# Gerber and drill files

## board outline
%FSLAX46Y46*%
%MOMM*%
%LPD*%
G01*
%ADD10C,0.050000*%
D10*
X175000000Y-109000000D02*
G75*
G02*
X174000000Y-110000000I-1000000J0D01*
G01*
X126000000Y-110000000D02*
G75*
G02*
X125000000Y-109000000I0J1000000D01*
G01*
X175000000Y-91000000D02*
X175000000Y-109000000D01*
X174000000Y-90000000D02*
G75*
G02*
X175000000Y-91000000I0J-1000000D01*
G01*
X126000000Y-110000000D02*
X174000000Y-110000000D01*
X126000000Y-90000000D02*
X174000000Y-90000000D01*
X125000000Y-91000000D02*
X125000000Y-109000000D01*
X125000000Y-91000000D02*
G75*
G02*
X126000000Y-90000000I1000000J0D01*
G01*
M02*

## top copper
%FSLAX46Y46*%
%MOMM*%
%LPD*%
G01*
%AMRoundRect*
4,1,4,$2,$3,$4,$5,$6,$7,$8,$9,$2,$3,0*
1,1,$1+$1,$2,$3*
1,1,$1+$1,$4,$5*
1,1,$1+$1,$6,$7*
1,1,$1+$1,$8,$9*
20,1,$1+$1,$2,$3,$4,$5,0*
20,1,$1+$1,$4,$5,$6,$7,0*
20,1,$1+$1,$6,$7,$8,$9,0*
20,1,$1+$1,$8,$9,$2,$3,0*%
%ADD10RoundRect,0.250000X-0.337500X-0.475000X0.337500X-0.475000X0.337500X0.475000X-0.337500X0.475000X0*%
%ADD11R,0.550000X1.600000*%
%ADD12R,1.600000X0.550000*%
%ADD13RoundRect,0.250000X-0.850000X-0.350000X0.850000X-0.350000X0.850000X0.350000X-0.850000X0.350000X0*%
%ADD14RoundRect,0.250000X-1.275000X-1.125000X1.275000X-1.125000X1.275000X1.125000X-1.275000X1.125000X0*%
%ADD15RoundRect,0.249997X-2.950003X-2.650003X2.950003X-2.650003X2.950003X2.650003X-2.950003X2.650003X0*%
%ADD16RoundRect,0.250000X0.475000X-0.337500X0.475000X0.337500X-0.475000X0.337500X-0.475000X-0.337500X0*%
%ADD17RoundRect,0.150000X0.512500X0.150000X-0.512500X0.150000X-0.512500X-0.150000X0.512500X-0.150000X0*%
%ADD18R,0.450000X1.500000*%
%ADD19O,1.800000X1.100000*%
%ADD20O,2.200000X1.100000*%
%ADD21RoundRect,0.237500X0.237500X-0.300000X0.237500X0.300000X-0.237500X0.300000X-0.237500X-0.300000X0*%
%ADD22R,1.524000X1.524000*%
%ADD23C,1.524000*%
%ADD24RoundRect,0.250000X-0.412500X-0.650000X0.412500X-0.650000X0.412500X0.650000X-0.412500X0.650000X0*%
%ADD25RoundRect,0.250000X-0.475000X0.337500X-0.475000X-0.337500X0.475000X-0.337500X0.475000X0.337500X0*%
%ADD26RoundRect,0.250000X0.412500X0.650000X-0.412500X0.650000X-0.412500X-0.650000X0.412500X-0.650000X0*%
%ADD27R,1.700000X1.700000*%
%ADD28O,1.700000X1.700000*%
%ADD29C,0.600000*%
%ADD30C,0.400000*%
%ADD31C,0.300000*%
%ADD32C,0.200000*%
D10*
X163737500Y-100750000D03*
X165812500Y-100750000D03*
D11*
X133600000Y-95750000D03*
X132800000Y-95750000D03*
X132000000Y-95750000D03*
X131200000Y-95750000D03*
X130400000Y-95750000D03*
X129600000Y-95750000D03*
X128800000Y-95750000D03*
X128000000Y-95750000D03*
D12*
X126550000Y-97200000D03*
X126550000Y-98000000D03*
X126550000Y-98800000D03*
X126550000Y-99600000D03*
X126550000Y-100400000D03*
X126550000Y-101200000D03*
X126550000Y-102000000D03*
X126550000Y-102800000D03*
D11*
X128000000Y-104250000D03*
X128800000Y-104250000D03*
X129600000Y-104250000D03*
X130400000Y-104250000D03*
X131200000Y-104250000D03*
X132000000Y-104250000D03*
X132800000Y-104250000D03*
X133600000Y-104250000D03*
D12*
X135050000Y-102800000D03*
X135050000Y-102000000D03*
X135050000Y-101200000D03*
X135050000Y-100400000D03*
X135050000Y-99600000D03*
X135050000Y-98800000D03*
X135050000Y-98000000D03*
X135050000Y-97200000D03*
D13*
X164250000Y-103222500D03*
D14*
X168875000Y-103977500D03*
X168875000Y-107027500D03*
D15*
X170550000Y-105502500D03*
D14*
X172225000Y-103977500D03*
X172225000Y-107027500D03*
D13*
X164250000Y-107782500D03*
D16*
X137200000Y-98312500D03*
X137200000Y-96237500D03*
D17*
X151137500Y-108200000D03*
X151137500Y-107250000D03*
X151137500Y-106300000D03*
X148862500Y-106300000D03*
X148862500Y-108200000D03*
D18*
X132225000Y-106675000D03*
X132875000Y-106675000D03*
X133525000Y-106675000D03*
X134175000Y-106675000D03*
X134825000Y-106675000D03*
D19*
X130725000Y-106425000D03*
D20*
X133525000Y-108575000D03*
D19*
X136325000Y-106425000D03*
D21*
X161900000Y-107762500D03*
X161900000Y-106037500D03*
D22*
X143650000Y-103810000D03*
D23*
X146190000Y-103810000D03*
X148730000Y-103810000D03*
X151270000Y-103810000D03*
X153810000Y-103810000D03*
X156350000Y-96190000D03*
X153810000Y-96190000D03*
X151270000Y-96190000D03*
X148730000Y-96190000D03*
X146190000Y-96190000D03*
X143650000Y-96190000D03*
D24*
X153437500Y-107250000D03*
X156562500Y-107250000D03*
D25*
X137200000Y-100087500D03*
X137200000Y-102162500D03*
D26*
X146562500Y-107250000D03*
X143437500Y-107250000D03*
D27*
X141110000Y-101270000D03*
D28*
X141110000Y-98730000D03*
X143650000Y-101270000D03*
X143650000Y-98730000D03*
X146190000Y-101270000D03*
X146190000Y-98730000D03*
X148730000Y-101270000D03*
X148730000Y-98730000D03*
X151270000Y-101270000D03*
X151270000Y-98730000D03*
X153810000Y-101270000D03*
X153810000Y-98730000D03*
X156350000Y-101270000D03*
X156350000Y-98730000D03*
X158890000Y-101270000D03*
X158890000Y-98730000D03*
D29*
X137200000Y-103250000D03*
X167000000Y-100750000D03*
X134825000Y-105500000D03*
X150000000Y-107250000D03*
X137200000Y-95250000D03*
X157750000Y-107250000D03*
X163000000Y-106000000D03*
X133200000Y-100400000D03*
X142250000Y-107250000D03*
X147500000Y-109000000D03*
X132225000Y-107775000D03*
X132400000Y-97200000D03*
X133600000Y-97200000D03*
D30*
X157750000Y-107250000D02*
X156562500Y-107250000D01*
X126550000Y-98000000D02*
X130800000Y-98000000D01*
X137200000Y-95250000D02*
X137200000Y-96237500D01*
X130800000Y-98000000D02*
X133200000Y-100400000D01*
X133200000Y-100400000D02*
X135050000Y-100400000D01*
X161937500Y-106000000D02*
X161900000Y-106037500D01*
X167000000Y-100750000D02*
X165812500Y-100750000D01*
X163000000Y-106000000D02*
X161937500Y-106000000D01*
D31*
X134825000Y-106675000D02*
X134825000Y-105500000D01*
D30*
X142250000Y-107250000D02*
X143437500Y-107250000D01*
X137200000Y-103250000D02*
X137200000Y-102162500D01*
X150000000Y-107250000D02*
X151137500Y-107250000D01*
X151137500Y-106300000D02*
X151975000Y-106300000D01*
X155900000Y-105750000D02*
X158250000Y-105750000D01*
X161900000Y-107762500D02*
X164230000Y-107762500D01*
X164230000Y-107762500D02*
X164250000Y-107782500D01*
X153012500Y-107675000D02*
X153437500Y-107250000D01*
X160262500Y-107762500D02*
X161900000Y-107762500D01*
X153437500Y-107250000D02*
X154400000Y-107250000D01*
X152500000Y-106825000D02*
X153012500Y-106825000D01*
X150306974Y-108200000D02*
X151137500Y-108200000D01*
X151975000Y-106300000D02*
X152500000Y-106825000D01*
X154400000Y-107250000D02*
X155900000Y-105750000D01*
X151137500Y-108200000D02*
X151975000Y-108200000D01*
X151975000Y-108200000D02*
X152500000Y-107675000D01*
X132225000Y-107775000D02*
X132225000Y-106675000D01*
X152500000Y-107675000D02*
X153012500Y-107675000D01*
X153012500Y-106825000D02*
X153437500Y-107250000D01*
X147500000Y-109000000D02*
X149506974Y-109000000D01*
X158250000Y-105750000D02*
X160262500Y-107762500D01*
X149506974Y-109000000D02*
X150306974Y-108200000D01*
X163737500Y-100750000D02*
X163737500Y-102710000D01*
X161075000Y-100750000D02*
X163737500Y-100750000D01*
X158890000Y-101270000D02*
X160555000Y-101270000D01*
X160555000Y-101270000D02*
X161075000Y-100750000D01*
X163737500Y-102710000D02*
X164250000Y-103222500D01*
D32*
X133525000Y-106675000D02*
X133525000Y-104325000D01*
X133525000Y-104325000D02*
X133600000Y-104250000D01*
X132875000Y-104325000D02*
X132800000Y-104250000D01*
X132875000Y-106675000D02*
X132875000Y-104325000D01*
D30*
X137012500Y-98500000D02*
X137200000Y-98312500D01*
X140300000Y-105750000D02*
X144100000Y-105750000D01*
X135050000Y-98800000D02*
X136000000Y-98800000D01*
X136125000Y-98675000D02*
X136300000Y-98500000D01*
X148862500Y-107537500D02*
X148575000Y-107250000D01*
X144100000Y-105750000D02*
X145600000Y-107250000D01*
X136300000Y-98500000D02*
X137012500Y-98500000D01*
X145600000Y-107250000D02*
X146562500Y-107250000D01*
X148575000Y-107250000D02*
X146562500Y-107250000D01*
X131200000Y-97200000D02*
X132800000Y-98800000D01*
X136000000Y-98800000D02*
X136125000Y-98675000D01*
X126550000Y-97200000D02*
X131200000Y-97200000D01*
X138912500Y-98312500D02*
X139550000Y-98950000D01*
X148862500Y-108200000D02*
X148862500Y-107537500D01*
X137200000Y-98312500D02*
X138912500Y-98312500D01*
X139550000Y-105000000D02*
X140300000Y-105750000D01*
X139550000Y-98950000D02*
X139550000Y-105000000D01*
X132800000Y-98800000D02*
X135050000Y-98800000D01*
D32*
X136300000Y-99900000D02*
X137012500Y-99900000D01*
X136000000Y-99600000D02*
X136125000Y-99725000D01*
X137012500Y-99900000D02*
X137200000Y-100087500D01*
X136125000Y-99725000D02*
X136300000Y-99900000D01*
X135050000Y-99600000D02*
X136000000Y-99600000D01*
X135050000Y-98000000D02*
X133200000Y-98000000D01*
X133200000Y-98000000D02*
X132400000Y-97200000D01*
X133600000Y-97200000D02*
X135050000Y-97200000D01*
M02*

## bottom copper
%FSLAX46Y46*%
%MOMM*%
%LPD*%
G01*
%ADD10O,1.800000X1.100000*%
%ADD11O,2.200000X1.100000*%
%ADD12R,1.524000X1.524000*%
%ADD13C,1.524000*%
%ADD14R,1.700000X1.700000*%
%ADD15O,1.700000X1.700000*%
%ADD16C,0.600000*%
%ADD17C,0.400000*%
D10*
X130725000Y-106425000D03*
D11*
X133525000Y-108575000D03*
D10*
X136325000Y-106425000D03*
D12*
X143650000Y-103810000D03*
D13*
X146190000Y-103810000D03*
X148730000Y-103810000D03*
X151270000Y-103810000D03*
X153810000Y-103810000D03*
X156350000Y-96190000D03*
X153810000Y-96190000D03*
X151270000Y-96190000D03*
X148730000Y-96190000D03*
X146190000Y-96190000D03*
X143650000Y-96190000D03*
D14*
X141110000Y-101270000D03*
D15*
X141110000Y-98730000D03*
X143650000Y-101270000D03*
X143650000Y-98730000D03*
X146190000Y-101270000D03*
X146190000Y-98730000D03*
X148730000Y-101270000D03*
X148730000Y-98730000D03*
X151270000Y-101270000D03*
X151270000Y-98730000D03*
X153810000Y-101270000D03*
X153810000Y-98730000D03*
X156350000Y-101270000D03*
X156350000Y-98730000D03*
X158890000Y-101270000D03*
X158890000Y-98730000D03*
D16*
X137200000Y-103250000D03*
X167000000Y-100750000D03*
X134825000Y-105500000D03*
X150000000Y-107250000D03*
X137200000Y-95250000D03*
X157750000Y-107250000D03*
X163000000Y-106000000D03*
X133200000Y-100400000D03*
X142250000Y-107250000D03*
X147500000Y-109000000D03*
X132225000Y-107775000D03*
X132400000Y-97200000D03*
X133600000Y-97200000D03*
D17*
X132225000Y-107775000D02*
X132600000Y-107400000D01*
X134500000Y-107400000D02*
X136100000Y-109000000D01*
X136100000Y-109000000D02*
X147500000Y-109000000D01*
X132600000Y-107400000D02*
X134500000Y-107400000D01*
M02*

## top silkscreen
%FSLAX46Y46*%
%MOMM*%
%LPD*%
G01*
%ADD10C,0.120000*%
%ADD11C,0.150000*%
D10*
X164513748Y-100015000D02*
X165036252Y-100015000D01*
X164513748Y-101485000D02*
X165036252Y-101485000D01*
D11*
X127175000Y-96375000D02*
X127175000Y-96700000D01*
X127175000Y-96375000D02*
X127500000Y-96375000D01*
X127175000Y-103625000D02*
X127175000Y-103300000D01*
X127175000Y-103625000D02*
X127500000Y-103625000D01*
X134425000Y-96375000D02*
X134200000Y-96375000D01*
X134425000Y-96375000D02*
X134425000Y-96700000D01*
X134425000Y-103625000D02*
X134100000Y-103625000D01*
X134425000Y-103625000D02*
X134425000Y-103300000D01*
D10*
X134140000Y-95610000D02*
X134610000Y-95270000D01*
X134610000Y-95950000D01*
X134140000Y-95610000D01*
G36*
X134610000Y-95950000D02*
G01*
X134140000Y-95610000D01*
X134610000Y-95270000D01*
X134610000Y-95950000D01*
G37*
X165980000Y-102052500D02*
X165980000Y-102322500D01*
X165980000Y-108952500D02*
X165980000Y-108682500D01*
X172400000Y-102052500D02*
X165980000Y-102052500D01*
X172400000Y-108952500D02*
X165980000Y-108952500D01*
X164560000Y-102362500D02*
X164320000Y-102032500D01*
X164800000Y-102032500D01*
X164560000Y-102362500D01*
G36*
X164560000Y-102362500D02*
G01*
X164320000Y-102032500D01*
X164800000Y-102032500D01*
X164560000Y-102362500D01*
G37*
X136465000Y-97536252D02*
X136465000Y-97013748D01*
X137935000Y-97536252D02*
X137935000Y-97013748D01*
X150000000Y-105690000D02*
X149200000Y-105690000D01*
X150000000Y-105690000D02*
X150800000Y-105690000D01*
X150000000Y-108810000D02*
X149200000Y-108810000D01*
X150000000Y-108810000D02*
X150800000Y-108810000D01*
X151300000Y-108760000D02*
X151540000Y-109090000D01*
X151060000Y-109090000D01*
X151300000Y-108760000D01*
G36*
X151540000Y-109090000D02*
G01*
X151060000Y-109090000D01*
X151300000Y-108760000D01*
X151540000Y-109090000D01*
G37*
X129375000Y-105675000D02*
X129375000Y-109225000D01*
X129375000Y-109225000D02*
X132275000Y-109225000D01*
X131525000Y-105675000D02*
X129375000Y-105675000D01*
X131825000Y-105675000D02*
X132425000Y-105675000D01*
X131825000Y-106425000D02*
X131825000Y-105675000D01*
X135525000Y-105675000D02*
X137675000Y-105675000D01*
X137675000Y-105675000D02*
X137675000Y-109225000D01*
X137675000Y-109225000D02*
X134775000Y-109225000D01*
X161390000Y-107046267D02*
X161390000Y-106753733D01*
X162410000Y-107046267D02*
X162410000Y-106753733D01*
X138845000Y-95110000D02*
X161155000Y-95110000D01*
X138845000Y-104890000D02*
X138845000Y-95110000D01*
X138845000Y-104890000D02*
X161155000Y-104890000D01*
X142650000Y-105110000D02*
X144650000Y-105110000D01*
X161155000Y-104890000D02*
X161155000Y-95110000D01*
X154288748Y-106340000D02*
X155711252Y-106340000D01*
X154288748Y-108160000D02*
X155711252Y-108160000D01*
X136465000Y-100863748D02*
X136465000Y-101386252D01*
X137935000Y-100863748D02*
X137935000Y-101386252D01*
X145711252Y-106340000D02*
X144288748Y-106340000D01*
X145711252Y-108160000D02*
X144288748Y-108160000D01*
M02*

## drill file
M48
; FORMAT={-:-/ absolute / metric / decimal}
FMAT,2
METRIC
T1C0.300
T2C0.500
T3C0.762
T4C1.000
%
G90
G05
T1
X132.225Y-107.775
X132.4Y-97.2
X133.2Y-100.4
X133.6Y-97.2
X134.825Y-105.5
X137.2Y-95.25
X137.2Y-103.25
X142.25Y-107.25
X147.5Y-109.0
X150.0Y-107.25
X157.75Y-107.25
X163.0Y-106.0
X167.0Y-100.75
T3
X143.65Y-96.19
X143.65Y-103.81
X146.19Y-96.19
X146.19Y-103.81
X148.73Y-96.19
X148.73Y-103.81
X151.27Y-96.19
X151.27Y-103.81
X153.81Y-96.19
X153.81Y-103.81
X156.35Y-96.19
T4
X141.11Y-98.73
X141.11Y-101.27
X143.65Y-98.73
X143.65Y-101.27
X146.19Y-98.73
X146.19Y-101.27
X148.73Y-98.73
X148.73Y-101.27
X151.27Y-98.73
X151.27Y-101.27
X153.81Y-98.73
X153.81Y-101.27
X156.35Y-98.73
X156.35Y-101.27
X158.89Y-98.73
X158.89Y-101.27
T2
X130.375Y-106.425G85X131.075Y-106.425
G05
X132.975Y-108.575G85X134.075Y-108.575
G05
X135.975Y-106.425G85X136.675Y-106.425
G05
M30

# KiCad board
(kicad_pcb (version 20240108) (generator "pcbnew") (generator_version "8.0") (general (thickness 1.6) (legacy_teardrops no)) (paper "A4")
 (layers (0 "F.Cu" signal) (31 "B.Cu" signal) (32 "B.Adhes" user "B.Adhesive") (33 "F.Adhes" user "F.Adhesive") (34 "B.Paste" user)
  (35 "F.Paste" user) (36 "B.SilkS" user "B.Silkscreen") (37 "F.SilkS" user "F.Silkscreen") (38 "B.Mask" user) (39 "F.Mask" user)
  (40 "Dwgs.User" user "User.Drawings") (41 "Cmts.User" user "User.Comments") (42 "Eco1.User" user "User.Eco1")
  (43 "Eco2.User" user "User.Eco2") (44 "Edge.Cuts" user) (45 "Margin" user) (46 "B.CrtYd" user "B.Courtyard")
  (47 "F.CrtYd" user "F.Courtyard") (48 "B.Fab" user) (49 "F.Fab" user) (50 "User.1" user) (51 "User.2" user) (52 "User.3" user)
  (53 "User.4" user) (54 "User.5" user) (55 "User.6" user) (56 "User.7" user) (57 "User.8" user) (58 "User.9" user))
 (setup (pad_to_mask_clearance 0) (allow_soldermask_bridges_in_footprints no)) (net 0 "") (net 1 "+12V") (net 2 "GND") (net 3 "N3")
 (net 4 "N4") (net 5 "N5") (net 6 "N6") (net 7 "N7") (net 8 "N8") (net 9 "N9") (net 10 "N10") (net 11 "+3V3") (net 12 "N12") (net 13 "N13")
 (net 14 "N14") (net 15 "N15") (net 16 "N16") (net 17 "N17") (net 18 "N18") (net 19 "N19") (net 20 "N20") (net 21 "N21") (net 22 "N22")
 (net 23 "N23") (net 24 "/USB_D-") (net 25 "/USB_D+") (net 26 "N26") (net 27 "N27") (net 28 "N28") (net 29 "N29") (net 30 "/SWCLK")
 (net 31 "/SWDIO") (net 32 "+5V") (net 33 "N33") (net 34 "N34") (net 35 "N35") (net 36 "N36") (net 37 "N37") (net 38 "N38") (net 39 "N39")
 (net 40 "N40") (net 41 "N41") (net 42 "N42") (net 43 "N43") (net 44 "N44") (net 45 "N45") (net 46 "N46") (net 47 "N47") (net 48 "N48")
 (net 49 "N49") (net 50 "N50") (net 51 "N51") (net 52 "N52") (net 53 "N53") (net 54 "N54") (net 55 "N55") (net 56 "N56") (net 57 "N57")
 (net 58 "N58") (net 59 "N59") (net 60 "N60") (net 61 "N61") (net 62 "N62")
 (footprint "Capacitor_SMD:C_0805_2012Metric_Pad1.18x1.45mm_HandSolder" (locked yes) (layer "F.Cu") (at 164.775 100.75)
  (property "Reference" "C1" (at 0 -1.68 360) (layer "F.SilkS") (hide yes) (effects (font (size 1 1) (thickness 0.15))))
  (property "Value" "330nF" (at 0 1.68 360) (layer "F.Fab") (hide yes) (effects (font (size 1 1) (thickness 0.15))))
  (fp_line (start -0.261252 -0.735) (end 0.261252 -0.735) (stroke (width 0.12) (type solid)) (layer "F.SilkS"))
  (fp_line (start -0.261252 0.735) (end 0.261252 0.735) (stroke (width 0.12) (type solid)) (layer "F.SilkS"))
  (pad "1" smd roundrect (at -1.0375 0) (size 1.175 1.45) (layers "F.Cu" "F.Paste" "F.Mask") (roundrect_rratio 0.212766) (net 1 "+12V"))
  (pad "2" smd roundrect (at 1.0375 0) (size 1.175 1.45) (layers "F.Cu" "F.Paste" "F.Mask") (roundrect_rratio 0.212766) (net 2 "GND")))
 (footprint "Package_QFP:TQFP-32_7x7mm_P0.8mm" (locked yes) (layer "F.Cu") (at 130.8 100 -90)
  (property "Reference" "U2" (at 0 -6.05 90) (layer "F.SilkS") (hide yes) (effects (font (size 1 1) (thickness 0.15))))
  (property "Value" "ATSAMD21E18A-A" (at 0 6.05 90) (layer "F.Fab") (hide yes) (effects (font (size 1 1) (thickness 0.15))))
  (fp_line (start -3.625 3.625) (end -3.3 3.625) (stroke (width 0.15) (type solid)) (layer "F.SilkS"))
  (fp_line (start -3.625 3.625) (end -3.625 3.3) (stroke (width 0.15) (type solid)) (layer "F.SilkS"))
  (fp_line (start 3.625 3.625) (end 3.3 3.625) (stroke (width 0.15) (type solid)) (layer "F.SilkS"))
  (fp_line (start 3.625 3.625) (end 3.625 3.3) (stroke (width 0.15) (type solid)) (layer "F.SilkS"))
  (fp_line (start -3.625 -3.625) (end -3.625 -3.4) (stroke (width 0.15) (type solid)) (layer "F.SilkS"))
  (fp_line (start -3.625 -3.625) (end -3.3 -3.625) (stroke (width 0.15) (type solid)) (layer "F.SilkS"))
  (fp_line (start 3.625 -3.625) (end 3.625 -3.3) (stroke (width 0.15) (type solid)) (layer "F.SilkS"))
  (fp_line (start 3.625 -3.625) (end 3.3 -3.625) (stroke (width 0.15) (type solid)) (layer "F.SilkS"))
  (fp_poly
   (pts (xy -4.39 -3.34) (xy -4.73 -3.81) (xy -4.05 -3.81) (xy -4.39 -3.34)) (stroke (width 0.12) (type solid)) (fill solid)
   (layer "F.SilkS"))
  (pad "1" smd rect (at -4.25 -2.8 270) (size 1.6 0.55) (layers "F.Cu" "F.Paste" "F.Mask") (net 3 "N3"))
  (pad "2" smd rect (at -4.25 -2 270) (size 1.6 0.55) (layers "F.Cu" "F.Paste" "F.Mask") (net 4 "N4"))
  (pad "3" smd rect (at -4.25 -1.2 270) (size 1.6 0.55) (layers "F.Cu" "F.Paste" "F.Mask") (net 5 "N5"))
  (pad "4" smd rect (at -4.25 -0.4 270) (size 1.6 0.55) (layers "F.Cu" "F.Paste" "F.Mask") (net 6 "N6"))
  (pad "5" smd rect (at -4.25 0.4 270) (size 1.6 0.55) (layers "F.Cu" "F.Paste" "F.Mask") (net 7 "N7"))
  (pad "6" smd rect (at -4.25 1.2 270) (size 1.6 0.55) (layers "F.Cu" "F.Paste" "F.Mask") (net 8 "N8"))
  (pad "7" smd rect (at -4.25 2 270) (size 1.6 0.55) (layers "F.Cu" "F.Paste" "F.Mask") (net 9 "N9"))
  (pad "8" smd rect (at -4.25 2.8 270) (size 1.6 0.55) (layers "F.Cu" "F.Paste" "F.Mask") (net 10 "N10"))
  (pad "9" smd rect (at -2.8 4.25) (size 1.6 0.55) (layers "F.Cu" "F.Paste" "F.Mask") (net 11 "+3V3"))
  (pad "10" smd rect (at -2 4.25) (size 1.6 0.55) (layers "F.Cu" "F.Paste" "F.Mask") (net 2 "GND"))
  (pad "11" smd rect (at -1.2 4.25) (size 1.6 0.55) (layers "F.Cu" "F.Paste" "F.Mask") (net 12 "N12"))
  (pad "12" smd rect (at -0.4 4.25) (size 1.6 0.55) (layers "F.Cu" "F.Paste" "F.Mask") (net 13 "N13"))
  (pad "13" smd rect (at 0.4 4.25) (size 1.6 0.55) (layers "F.Cu" "F.Paste" "F.Mask") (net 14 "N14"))
  (pad "14" smd rect (at 1.2 4.25) (size 1.6 0.55) (layers "F.Cu" "F.Paste" "F.Mask") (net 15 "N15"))
  (pad "15" smd rect (at 2 4.25) (size 1.6 0.55) (layers "F.Cu" "F.Paste" "F.Mask") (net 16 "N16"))
  (pad "16" smd rect (at 2.8 4.25) (size 1.6 0.55) (layers "F.Cu" "F.Paste" "F.Mask") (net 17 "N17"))
  (pad "17" smd rect (at 4.25 2.8 270) (size 1.6 0.55) (layers "F.Cu" "F.Paste" "F.Mask") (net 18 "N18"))
  (pad "18" smd rect (at 4.25 2 270) (size 1.6 0.55) (layers "F.Cu" "F.Paste" "F.Mask") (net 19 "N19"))
  (pad "19" smd rect (at 4.25 1.2 270) (size 1.6 0.55) (layers "F.Cu" "F.Paste" "F.Mask") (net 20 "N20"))
  (pad "20" smd rect (at 4.25 0.4 270) (size 1.6 0.55) (layers "F.Cu" "F.Paste" "F.Mask") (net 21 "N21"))
  (pad "21" smd rect (at 4.25 -0.4 270) (size 1.6 0.55) (layers "F.Cu" "F.Paste" "F.Mask") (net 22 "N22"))
  (pad "22" smd rect (at 4.25 -1.2 270) (size 1.6 0.55) (layers "F.Cu" "F.Paste" "F.Mask") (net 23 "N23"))
  (pad "23" smd rect (at 4.25 -2 270) (size 1.6 0.55) (layers "F.Cu" "F.Paste" "F.Mask") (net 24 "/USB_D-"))
  (pad "24" smd rect (at 4.25 -2.8 270) (size 1.6 0.55) (layers "F.Cu" "F.Paste" "F.Mask") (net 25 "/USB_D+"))
  (pad "25" smd rect (at 2.8 -4.25) (size 1.6 0.55) (layers "F.Cu" "F.Paste" "F.Mask") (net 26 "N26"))
  (pad "26" smd rect (at 2 -4.25) (size 1.6 0.55) (layers "F.Cu" "F.Paste" "F.Mask") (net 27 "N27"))
  (pad "27" smd rect (at 1.2 -4.25) (size 1.6 0.55) (layers "F.Cu" "F.Paste" "F.Mask") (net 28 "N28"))
  (pad "28" smd rect (at 0.4 -4.25) (size 1.6 0.55) (layers "F.Cu" "F.Paste" "F.Mask") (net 2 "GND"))
  (pad "29" smd rect (at -0.4 -4.25) (size 1.6 0.55) (layers "F.Cu" "F.Paste" "F.Mask") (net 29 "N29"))
  (pad "30" smd rect (at -1.2 -4.25) (size 1.6 0.55) (layers "F.Cu" "F.Paste" "F.Mask") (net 11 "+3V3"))
  (pad "31" smd rect (at -2 -4.25) (size 1.6 0.55) (layers "F.Cu" "F.Paste" "F.Mask") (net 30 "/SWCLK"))
  (pad "32" smd rect (at -2.8 -4.25) (size 1.6 0.55) (layers "F.Cu" "F.Paste" "F.Mask") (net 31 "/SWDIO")))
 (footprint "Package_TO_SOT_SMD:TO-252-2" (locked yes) (layer "F.Cu") (at 169.29 105.5025)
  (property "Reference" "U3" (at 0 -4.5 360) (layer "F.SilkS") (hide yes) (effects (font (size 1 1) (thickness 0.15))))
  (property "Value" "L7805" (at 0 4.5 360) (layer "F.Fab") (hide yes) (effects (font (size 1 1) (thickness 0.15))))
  (fp_line (start -3.31 -3.45) (end -3.31 -3.18) (stroke (width 0.12) (type solid)) (layer "F.SilkS"))
  (fp_line (start -3.31 3.45) (end -3.31 3.18) (stroke (width 0.12) (type solid)) (layer "F.SilkS"))
  (fp_line (start 3.11 -3.45) (end -3.31 -3.45) (stroke (width 0.12) (type solid)) (layer "F.SilkS"))
  (fp_line (start 3.11 3.45) (end -3.31 3.45) (stroke (width 0.12) (type solid)) (layer "F.SilkS"))
  (fp_poly
   (pts (xy -4.73 -3.14) (xy -4.97 -3.47) (xy -4.49 -3.47) (xy -4.73 -3.14)) (stroke (width 0.12) (type solid)) (fill solid)
   (layer "F.SilkS"))
  (pad "1" smd roundrect (at -5.04 -2.28) (size 2.2 1.2) (layers "F.Cu" "F.Paste" "F.Mask") (roundrect_rratio 0.208333) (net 1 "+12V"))
  (pad "2" smd roundrect (at -0.415 -1.525) (size 3.05 2.75) (layers "F.Cu" "F.Paste") (roundrect_rratio 0.090909) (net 2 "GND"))
  (pad "2" smd roundrect (at -0.415 1.525) (size 3.05 2.75) (layers "F.Cu" "F.Paste") (roundrect_rratio 0.090909) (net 2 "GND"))
  (pad "2" smd roundrect (at 1.26 0) (size 6.4 5.8) (layers "F.Cu" "F.Mask") (roundrect_rratio 0.043103) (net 2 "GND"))
  (pad "2" smd roundrect (at 2.935 -1.525) (size 3.05 2.75) (layers "F.Cu" "F.Paste") (roundrect_rratio 0.090909) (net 2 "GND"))
  (pad "2" smd roundrect (at 2.935 1.525) (size 3.05 2.75) (layers "F.Cu" "F.Paste") (roundrect_rratio 0.090909) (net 2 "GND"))
  (pad "3" smd roundrect (at -5.04 2.28) (size 2.2 1.2) (layers "F.Cu" "F.Paste" "F.Mask") (roundrect_rratio 0.208333) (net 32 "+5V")))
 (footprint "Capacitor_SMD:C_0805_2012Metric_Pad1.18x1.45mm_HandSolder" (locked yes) (layer "F.Cu") (at 137.2 97.275 90)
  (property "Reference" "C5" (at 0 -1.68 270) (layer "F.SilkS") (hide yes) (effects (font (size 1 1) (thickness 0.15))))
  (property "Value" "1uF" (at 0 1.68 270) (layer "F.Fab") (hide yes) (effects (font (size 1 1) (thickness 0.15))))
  (fp_line (start -0.261252 -0.735) (end 0.261252 -0.735) (stroke (width 0.12) (type solid)) (layer "F.SilkS"))
  (fp_line (start -0.261252 0.735) (end 0.261252 0.735) (stroke (width 0.12) (type solid)) (layer "F.SilkS"))
  (pad "1" smd roundrect (at -1.0375 0 90) (size 1.175 1.45) (layers "F.Cu" "F.Paste" "F.Mask") (roundrect_rratio 0.212766) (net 11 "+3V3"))
  (pad "2" smd roundrect (at 1.0375 0 90) (size 1.175 1.45) (layers "F.Cu" "F.Paste" "F.Mask") (roundrect_rratio 0.212766) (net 2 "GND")))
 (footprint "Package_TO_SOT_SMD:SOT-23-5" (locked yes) (layer "F.Cu") (at 150 107.25 180)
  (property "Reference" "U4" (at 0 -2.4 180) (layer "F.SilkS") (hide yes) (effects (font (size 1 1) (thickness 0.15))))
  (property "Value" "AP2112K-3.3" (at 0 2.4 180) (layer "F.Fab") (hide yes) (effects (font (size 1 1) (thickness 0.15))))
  (fp_line (start 0 1.56) (end 0.8 1.56) (stroke (width 0.12) (type solid)) (layer "F.SilkS"))
  (fp_line (start 0 1.56) (end -0.8 1.56) (stroke (width 0.12) (type solid)) (layer "F.SilkS"))
  (fp_line (start 0 -1.56) (end 0.8 -1.56) (stroke (width 0.12) (type solid)) (layer "F.SilkS"))
  (fp_line (start 0 -1.56) (end -0.8 -1.56) (stroke (width 0.12) (type solid)) (layer "F.SilkS"))
  (fp_poly
   (pts (xy -1.3 -1.51) (xy -1.54 -1.84) (xy -1.06 -1.84) (xy -1.3 -1.51)) (stroke (width 0.12) (type solid)) (fill solid) (layer "F.SilkS"))
  (pad "1" smd roundrect (at -1.1375 -0.95 180) (size 1.325 0.6) (layers "F.Cu" "F.Paste" "F.Mask") (roundrect_rratio 0.25) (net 32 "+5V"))
  (pad "2" smd roundrect (at -1.1375 0 180) (size 1.325 0.6) (layers "F.Cu" "F.Paste" "F.Mask") (roundrect_rratio 0.25) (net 2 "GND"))
  (pad "3" smd roundrect (at -1.1375 0.95 180) (size 1.325 0.6) (layers "F.Cu" "F.Paste" "F.Mask") (roundrect_rratio 0.25) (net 32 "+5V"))
  (pad "4" smd roundrect (at 1.1375 0.95 180) (size 1.325 0.6) (layers "F.Cu" "F.Paste" "F.Mask") (roundrect_rratio 0.25) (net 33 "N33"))
  (pad "5" smd roundrect (at 1.1375 -0.95 180) (size 1.325 0.6) (layers "F.Cu" "F.Paste" "F.Mask") (roundrect_rratio 0.25) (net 11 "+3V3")))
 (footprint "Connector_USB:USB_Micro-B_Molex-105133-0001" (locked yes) (layer "F.Cu") (at 133.525 107.5)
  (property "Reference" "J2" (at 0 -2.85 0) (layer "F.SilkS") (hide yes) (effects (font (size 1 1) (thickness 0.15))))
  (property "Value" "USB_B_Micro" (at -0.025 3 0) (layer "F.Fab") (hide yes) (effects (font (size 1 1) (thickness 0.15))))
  (fp_line (start -4.15 -1.825) (end -4.15 1.725) (stroke (width 0.12) (type solid)) (layer "F.SilkS"))
  (fp_line (start -4.15 1.725) (end -1.25 1.725) (stroke (width 0.12) (type solid)) (layer "F.SilkS"))
  (fp_line (start -2 -1.825) (end -4.15 -1.825) (stroke (width 0.12) (type solid)) (layer "F.SilkS"))
  (fp_line (start -1.7 -1.825) (end -1.1 -1.825) (stroke (width 0.12) (type solid)) (layer "F.SilkS"))
  (fp_line (start -1.7 -1.075) (end -1.7 -1.825) (stroke (width 0.12) (type solid)) (layer "F.SilkS"))
  (fp_line (start 2 -1.825) (end 4.15 -1.825) (stroke (width 0.12) (type solid)) (layer "F.SilkS"))
  (fp_line (start 4.15 -1.825) (end 4.15 1.725) (stroke (width 0.12) (type solid)) (layer "F.SilkS"))
  (fp_line (start 4.15 1.725) (end 1.25 1.725) (stroke (width 0.12) (type solid)) (layer "F.SilkS"))
  (pad "1" smd rect (at -1.3 -0.825) (size 0.45 1.5) (layers "F.Cu" "F.Paste" "F.Mask") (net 32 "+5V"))
  (pad "2" smd rect (at -0.65 -0.825) (size 0.45 1.5) (layers "F.Cu" "F.Paste" "F.Mask") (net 24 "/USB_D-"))
  (pad "3" smd rect (at 0 -0.825) (size 0.45 1.5) (layers "F.Cu" "F.Paste" "F.Mask") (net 25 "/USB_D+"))
  (pad "4" smd rect (at 0.65 -0.825) (size 0.45 1.5) (layers "F.Cu" "F.Paste" "F.Mask") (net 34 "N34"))
  (pad "5" smd rect (at 1.3 -0.825) (size 0.45 1.5) (layers "F.Cu" "F.Paste" "F.Mask") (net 2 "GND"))
  (pad "6" thru_hole oval (at -2.8 -1.075) (size 1.8 1.1) (drill oval 1.2 0.5) (layers "*.Cu" "*.Mask") (remove_unused_layers no)
   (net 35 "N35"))
  (pad "6" thru_hole oval (at 0 1.075) (size 2.2 1.1) (drill oval 1.6 0.5) (layers "*.Cu" "*.Mask") (remove_unused_layers no) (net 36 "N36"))
  (pad "6" thru_hole oval (at 2.8 -1.075) (size 1.8 1.1) (drill oval 1.2 0.5) (layers "*.Cu" "*.Mask") (remove_unused_layers no)
   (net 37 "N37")))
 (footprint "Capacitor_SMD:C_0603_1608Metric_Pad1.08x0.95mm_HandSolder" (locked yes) (layer "F.Cu") (at 161.9 106.9 90)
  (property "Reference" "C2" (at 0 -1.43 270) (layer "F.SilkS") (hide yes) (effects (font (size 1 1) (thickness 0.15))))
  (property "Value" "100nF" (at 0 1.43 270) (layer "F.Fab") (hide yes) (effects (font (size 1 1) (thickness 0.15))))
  (fp_line (start -0.146267 -0.51) (end 0.146267 -0.51) (stroke (width 0.12) (type solid)) (layer "F.SilkS"))
  (fp_line (start -0.146267 0.51) (end 0.146267 0.51) (stroke (width 0.12) (type solid)) (layer "F.SilkS"))
  (pad "1" smd roundrect (at -0.8625 0 90) (size 1.075 0.95) (layers "F.Cu" "F.Paste" "F.Mask") (roundrect_rratio 0.25) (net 32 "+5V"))
  (pad "2" smd roundrect (at 0.8625 0 90) (size 1.075 0.95) (layers "F.Cu" "F.Paste" "F.Mask") (roundrect_rratio 0.25) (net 2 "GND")))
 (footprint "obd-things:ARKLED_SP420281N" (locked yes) (layer "F.Cu") (at 143.65 103.81 90)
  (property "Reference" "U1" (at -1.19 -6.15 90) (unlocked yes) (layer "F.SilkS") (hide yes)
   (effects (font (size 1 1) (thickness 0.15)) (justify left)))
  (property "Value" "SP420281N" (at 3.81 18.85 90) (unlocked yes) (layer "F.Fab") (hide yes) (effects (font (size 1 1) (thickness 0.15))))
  (fp_line (start 8.7 -4.805) (end 8.7 17.505) (stroke (width 0.12) (type default)) (layer "F.SilkS"))
  (fp_line (start -1.08 -4.805) (end 8.7 -4.805) (stroke (width 0.12) (type default)) (layer "F.SilkS"))
  (fp_line (start -1.08 -4.805) (end -1.08 17.505) (stroke (width 0.12) (type default)) (layer "F.SilkS"))
  (fp_line (start -1.3 -1) (end -1.3 1) (stroke (width 0.12) (type default)) (layer "F.SilkS"))
  (fp_line (start -1.08 17.505) (end 8.7 17.505) (stroke (width 0.12) (type default)) (layer "F.SilkS"))
  (pad "1" thru_hole rect (at 0 0 90) (size 1.524 1.524) (drill 0.762) (layers "*.Cu" "*.Mask") (remove_unused_layers no) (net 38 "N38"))
  (pad "2" thru_hole circle (at 0 2.54 90) (size 1.524 1.524) (drill 0.762) (layers "*.Cu" "*.Mask") (remove_unused_layers no)
   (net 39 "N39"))
  (pad "3" thru_hole circle (at 0 5.08 90) (size 1.524 1.524) (drill 0.762) (layers "*.Cu" "*.Mask") (remove_unused_layers no)
   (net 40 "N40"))
  (pad "4" thru_hole circle (at 0 7.62 90) (size 1.524 1.524) (drill 0.762) (layers "*.Cu" "*.Mask") (remove_unused_layers no)
   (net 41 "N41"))
  (pad "5" thru_hole circle (at 0 10.16 90) (size 1.524 1.524) (drill 0.762) (layers "*.Cu" "*.Mask") (remove_unused_layers no)
   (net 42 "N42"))
  (pad "7" thru_hole circle (at 7.62 12.7 90) (size 1.524 1.524) (drill 0.762) (layers "*.Cu" "*.Mask") (remove_unused_layers no)
   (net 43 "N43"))
  (pad "8" thru_hole circle (at 7.62 10.16 90) (size 1.524 1.524) (drill 0.762) (layers "*.Cu" "*.Mask") (remove_unused_layers no)
   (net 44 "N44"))
  (pad "9" thru_hole circle (at 7.62 7.62 90) (size 1.524 1.524) (drill 0.762) (layers "*.Cu" "*.Mask") (remove_unused_layers no)
   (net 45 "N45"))
  (pad "10" thru_hole circle (at 7.62 5.08 90) (size 1.524 1.524) (drill 0.762) (layers "*.Cu" "*.Mask") (remove_unused_layers no)
   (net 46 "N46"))
  (pad "11" thru_hole circle (at 7.62 2.54 90) (size 1.524 1.524) (drill 0.762) (layers "*.Cu" "*.Mask") (remove_unused_layers no)
   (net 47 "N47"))
  (pad "12" thru_hole circle (at 7.62 0 90) (size 1.524 1.524) (drill 0.762) (layers "*.Cu" "*.Mask") (remove_unused_layers no)
   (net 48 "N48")))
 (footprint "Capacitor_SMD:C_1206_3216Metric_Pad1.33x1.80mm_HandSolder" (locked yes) (layer "F.Cu") (at 155 107.25)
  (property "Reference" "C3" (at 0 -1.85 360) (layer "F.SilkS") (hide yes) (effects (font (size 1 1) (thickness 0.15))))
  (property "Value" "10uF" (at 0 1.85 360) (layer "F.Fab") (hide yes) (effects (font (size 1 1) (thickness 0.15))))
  (fp_line (start -0.711252 -0.91) (end 0.711252 -0.91) (stroke (width 0.12) (type solid)) (layer "F.SilkS"))
  (fp_line (start -0.711252 0.91) (end 0.711252 0.91) (stroke (width 0.12) (type solid)) (layer "F.SilkS"))
  (pad "1" smd roundrect (at -1.5625 0) (size 1.325 1.8) (layers "F.Cu" "F.Paste" "F.Mask") (roundrect_rratio 0.188679) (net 32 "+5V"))
  (pad "2" smd roundrect (at 1.5625 0) (size 1.325 1.8) (layers "F.Cu" "F.Paste" "F.Mask") (roundrect_rratio 0.188679) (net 2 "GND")))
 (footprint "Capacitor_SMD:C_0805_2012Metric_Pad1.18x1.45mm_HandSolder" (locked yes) (layer "F.Cu") (at 137.2 101.125 -90)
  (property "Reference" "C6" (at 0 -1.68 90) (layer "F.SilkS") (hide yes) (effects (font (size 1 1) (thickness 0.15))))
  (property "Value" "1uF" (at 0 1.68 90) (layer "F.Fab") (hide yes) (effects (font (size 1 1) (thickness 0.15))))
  (fp_line (start -0.261252 0.735) (end 0.261252 0.735) (stroke (width 0.12) (type solid)) (layer "F.SilkS"))
  (fp_line (start -0.261252 -0.735) (end 0.261252 -0.735) (stroke (width 0.12) (type solid)) (layer "F.SilkS"))
  (pad "1" smd roundrect (at -1.0375 0 270) (size 1.175 1.45) (layers "F.Cu" "F.Paste" "F.Mask") (roundrect_rratio 0.212766) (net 29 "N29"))
  (pad "2" smd roundrect (at 1.0375 0 270) (size 1.175 1.45) (layers "F.Cu" "F.Paste" "F.Mask") (roundrect_rratio 0.212766) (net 2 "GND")))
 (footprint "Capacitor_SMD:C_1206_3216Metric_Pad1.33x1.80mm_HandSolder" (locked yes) (layer "F.Cu") (at 145 107.25 180)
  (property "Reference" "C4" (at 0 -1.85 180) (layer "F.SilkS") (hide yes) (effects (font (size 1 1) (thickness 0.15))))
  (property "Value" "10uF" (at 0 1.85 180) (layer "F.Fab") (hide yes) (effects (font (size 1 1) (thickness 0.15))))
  (fp_line (start -0.711252 0.91) (end 0.711252 0.91) (stroke (width 0.12) (type solid)) (layer "F.SilkS"))
  (fp_line (start -0.711252 -0.91) (end 0.711252 -0.91) (stroke (width 0.12) (type solid)) (layer "F.SilkS"))
  (pad "1" smd roundrect (at -1.5625 0 180) (size 1.325 1.8) (layers "F.Cu" "F.Paste" "F.Mask") (roundrect_rratio 0.188679) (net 11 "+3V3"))
  (pad "2" smd roundrect (at 1.5625 0 180) (size 1.325 1.8) (layers "F.Cu" "F.Paste" "F.Mask") (roundrect_rratio 0.188679) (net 2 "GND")))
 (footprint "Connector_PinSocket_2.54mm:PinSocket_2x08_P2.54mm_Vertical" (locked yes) (layer "B.Cu") (at 141.11 101.27 -90)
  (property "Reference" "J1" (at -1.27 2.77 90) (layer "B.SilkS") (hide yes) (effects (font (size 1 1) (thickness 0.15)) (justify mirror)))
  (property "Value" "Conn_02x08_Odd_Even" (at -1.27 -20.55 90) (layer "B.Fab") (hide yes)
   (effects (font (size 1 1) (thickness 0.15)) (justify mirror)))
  (pad "1" thru_hole rect (at 0 0 270) (size 1.7 1.7) (drill 1) (layers "*.Cu" "*.Mask") (remove_unused_layers no) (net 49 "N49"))
  (pad "2" thru_hole oval (at -2.54 0 270) (size 1.7 1.7) (drill 1) (layers "*.Cu" "*.Mask") (remove_unused_layers no) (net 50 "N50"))
  (pad "3" thru_hole oval (at 0 -2.54 270) (size 1.7 1.7) (drill 1) (layers "*.Cu" "*.Mask") (remove_unused_layers no) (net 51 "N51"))
  (pad "4" thru_hole oval (at -2.54 -2.54 270) (size 1.7 1.7) (drill 1) (layers "*.Cu" "*.Mask") (remove_unused_layers no) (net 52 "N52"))
  (pad "5" thru_hole oval (at 0 -5.08 270) (size 1.7 1.7) (drill 1) (layers "*.Cu" "*.Mask") (remove_unused_layers no) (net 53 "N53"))
  (pad "6" thru_hole oval (at -2.54 -5.08 270) (size 1.7 1.7) (drill 1) (layers "*.Cu" "*.Mask") (remove_unused_layers no) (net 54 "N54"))
  (pad "7" thru_hole oval (at 0 -7.62 270) (size 1.7 1.7) (drill 1) (layers "*.Cu" "*.Mask") (remove_unused_layers no) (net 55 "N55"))
  (pad "8" thru_hole oval (at -2.54 -7.62 270) (size 1.7 1.7) (drill 1) (layers "*.Cu" "*.Mask") (remove_unused_layers no) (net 2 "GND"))
  (pad "9" thru_hole oval (at 0 -10.16 270) (size 1.7 1.7) (drill 1) (layers "*.Cu" "*.Mask") (remove_unused_layers no) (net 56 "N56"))
  (pad "10" thru_hole oval (at -2.54 -10.16 270) (size 1.7 1.7) (drill 1) (layers "*.Cu" "*.Mask") (remove_unused_layers no) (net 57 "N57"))
  (pad "11" thru_hole oval (at 0 -12.7 270) (size 1.7 1.7) (drill 1) (layers "*.Cu" "*.Mask") (remove_unused_layers no) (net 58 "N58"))
  (pad "12" thru_hole oval (at -2.54 -12.7 270) (size 1.7 1.7) (drill 1) (layers "*.Cu" "*.Mask") (remove_unused_layers no) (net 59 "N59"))
  (pad "13" thru_hole oval (at 0 -15.24 270) (size 1.7 1.7) (drill 1) (layers "*.Cu" "*.Mask") (remove_unused_layers no) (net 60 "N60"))
  (pad "14" thru_hole oval (at -2.54 -15.24 270) (size 1.7 1.7) (drill 1) (layers "*.Cu" "*.Mask") (remove_unused_layers no) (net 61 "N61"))
  (pad "15" thru_hole oval (at 0 -17.78 270) (size 1.7 1.7) (drill 1) (layers "*.Cu" "*.Mask") (remove_unused_layers no) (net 1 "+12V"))
  (pad "16" thru_hole oval (at -2.54 -17.78 270) (size 1.7 1.7) (drill 1) (layers "*.Cu" "*.Mask") (remove_unused_layers no) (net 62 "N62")))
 (gr_arc (start 175 109) (mid 174.707107 109.707107) (end 174 110) (locked yes) (stroke (width 0.05) (type default)) (layer "Edge.Cuts"))
 (gr_arc (start 126 110) (mid 125.292893 109.707107) (end 125 109) (locked yes) (stroke (width 0.05) (type default)) (layer "Edge.Cuts"))
 (gr_line (start 175 91) (end 175 109) (locked yes) (stroke (width 0.05) (type default)) (layer "Edge.Cuts"))
 (gr_arc (start 174 90) (mid 174.707107 90.292893) (end 175 91) (locked yes) (stroke (width 0.05) (type default)) (layer "Edge.Cuts"))
 (gr_line (start 126 110) (end 174 110) (locked yes) (stroke (width 0.05) (type default)) (layer "Edge.Cuts"))
 (gr_line (start 126 90) (end 174 90) (locked yes) (stroke (width 0.05) (type default)) (layer "Edge.Cuts"))
 (gr_line (start 125 91) (end 125 109) (locked yes) (stroke (width 0.05) (type default)) (layer "Edge.Cuts"))
 (gr_arc (start 125 91) (mid 125.292893 90.292893) (end 126 90) (locked yes) (stroke (width 0.05) (type default)) (layer "Edge.Cuts"))
 (segment (start 157.75 107.25) (end 156.5625 107.25) (width 0.4) (locked yes) (layer "F.Cu") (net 2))
 (segment (start 126.55 98) (end 130.8 98) (width 0.4) (locked yes) (layer "F.Cu") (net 2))
 (segment (start 137.2 95.25) (end 137.2 96.2375) (width 0.4) (locked yes) (layer "F.Cu") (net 2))
 (segment (start 130.8 98) (end 133.2 100.4) (width 0.4) (locked yes) (layer "F.Cu") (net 2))
 (segment (start 133.2 100.4) (end 135.05 100.4) (width 0.4) (locked yes) (layer "F.Cu") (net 2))
 (segment (start 161.9375 106) (end 161.9 106.0375) (width 0.4) (locked yes) (layer "F.Cu") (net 2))
 (segment (start 167 100.75) (end 165.8125 100.75) (width 0.4) (locked yes) (layer "F.Cu") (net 2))
 (segment (start 163 106) (end 161.9375 106) (width 0.4) (locked yes) (layer "F.Cu") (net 2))
 (segment (start 134.825 106.675) (end 134.825 105.5) (width 0.3) (locked yes) (layer "F.Cu") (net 2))
 (segment (start 142.25 107.25) (end 143.4375 107.25) (width 0.4) (locked yes) (layer "F.Cu") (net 2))
 (segment (start 137.2 103.25) (end 137.2 102.1625) (width 0.4) (locked yes) (layer "F.Cu") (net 2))
 (segment (start 150 107.25) (end 151.1375 107.25) (width 0.4) (locked yes) (layer "F.Cu") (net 2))
 (via (at 137.2 103.25) (size 0.6) (drill 0.3) (layers "F.Cu" "B.Cu") (locked yes) (free yes) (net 2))
 (via (at 167 100.75) (size 0.6) (drill 0.3) (layers "F.Cu" "B.Cu") (locked yes) (free yes) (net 2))
 (via (at 134.825 105.5) (size 0.6) (drill 0.3) (layers "F.Cu" "B.Cu") (locked yes) (free yes) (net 2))
 (via (at 150 107.25) (size 0.6) (drill 0.3) (layers "F.Cu" "B.Cu") (locked yes) (free yes) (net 2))
 (via (at 137.2 95.25) (size 0.6) (drill 0.3) (layers "F.Cu" "B.Cu") (locked yes) (free yes) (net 2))
 (via (at 157.75 107.25) (size 0.6) (drill 0.3) (layers "F.Cu" "B.Cu") (locked yes) (free yes) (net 2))
 (via (at 163 106) (size 0.6) (drill 0.3) (layers "F.Cu" "B.Cu") (locked yes) (free yes) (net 2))
 (via (at 133.2 100.4) (size 0.6) (drill 0.3) (layers "F.Cu" "B.Cu") (locked yes) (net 2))
 (via (at 142.25 107.25) (size 0.6) (drill 0.3) (layers "F.Cu" "B.Cu") (locked yes) (free yes) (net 2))
 (segment (start 151.1375 106.3) (end 151.975 106.3) (width 0.4) (locked yes) (layer "F.Cu") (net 32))
 (segment (start 155.9 105.75) (end 158.25 105.75) (width 0.4) (locked yes) (layer "F.Cu") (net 32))
 (segment (start 161.9 107.7625) (end 164.23 107.7625) (width 0.4) (locked yes) (layer "F.Cu") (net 32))
 (segment (start 164.23 107.7625) (end 164.25 107.7825) (width 0.4) (locked yes) (layer "F.Cu") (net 32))
 (segment (start 153.0125 107.675) (end 153.4375 107.25) (width 0.4) (locked yes) (layer "F.Cu") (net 32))
 (segment (start 160.2625 107.7625) (end 161.9 107.7625) (width 0.4) (locked yes) (layer "F.Cu") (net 32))
 (segment (start 153.4375 107.25) (end 154.4 107.25) (width 0.4) (locked yes) (layer "F.Cu") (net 32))
 (segment (start 152.5 106.825) (end 153.0125 106.825) (width 0.4) (locked yes) (layer "F.Cu") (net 32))
 (segment (start 150.306974 108.2) (end 151.1375 108.2) (width 0.4) (locked yes) (layer "F.Cu") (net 32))
 (segment (start 151.975 106.3) (end 152.5 106.825) (width 0.4) (locked yes) (layer "F.Cu") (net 32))
 (segment (start 154.4 107.25) (end 155.9 105.75) (width 0.4) (locked yes) (layer "F.Cu") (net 32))
 (segment (start 151.1375 108.2) (end 151.975 108.2) (width 0.4) (locked yes) (layer "F.Cu") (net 32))
 (segment (start 151.975 108.2) (end 152.5 107.675) (width 0.4) (locked yes) (layer "F.Cu") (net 32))
 (segment (start 132.225 107.775) (end 132.225 106.675) (width 0.4) (locked yes) (layer "F.Cu") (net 32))
 (segment (start 152.5 107.675) (end 153.0125 107.675) (width 0.4) (locked yes) (layer "F.Cu") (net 32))
 (segment (start 153.0125 106.825) (end 153.4375 107.25) (width 0.4) (locked yes) (layer "F.Cu") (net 32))
 (segment (start 147.5 109) (end 149.506974 109) (width 0.4) (locked yes) (layer "F.Cu") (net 32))
 (segment (start 158.25 105.75) (end 160.2625 107.7625) (width 0.4) (locked yes) (layer "F.Cu") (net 32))
 (segment (start 149.506974 109) (end 150.306974 108.2) (width 0.4) (locked yes) (layer "F.Cu") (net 32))
 (via (at 147.5 109) (size 0.6) (drill 0.3) (layers "F.Cu" "B.Cu") (locked yes) (free yes) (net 32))
 (via (at 132.225 107.775) (size 0.6) (drill 0.3) (layers "F.Cu" "B.Cu") (locked yes) (free yes) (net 32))
 (segment (start 132.225 107.775) (end 132.6 107.4) (width 0.4) (locked yes) (layer "B.Cu") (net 32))
 (segment (start 134.5 107.4) (end 136.1 109) (width 0.4) (locked yes) (layer "B.Cu") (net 32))
 (segment (start 136.1 109) (end 147.5 109) (width 0.4) (locked yes) (layer "B.Cu") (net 32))
 (segment (start 132.6 107.4) (end 134.5 107.4) (width 0.4) (locked yes) (layer "B.Cu") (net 32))
 (segment (start 163.7375 100.75) (end 163.7375 102.71) (width 0.4) (locked yes) (layer "F.Cu") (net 1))
 (segment (start 161.075 100.75) (end 163.7375 100.75) (width 0.4) (locked yes) (layer "F.Cu") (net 1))
 (segment (start 158.89 101.27) (end 160.555 101.27) (width 0.4) (locked yes) (layer "F.Cu") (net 1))
 (segment (start 160.555 101.27) (end 161.075 100.75) (width 0.4) (locked yes) (layer "F.Cu") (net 1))
 (segment (start 163.7375 102.71) (end 164.25 103.2225) (width 0.4) (locked yes) (layer "F.Cu") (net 1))
 (segment (start 133.525 106.675) (end 133.525 104.325) (width 0.2) (locked yes) (layer "F.Cu") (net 25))
 (segment (start 133.525 104.325) (end 133.6 104.25) (width 0.2) (locked yes) (layer "F.Cu") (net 25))
 (segment (start 132.875 104.325) (end 132.8 104.25) (width 0.2) (locked yes) (layer "F.Cu") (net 24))
 (segment (start 132.875 106.675) (end 132.875 104.325) (width 0.2) (locked yes) (layer "F.Cu") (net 24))
 (segment (start 137.0125 98.5) (end 137.2 98.3125) (width 0.4) (locked yes) (layer "F.Cu") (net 11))
 (segment (start 140.3 105.75) (end 144.1 105.75) (width 0.4) (locked yes) (layer "F.Cu") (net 11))
 (segment (start 135.05 98.8) (end 136 98.8) (width 0.4) (locked yes) (layer "F.Cu") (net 11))
 (segment (start 136.125 98.675) (end 136.3 98.5) (width 0.4) (locked yes) (layer "F.Cu") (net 11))
 (segment (start 148.8625 107.5375) (end 148.575 107.25) (width 0.4) (locked yes) (layer "F.Cu") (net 11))
 (segment (start 144.1 105.75) (end 145.6 107.25) (width 0.4) (locked yes) (layer "F.Cu") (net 11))
 (segment (start 136.3 98.5) (end 137.0125 98.5) (width 0.4) (locked yes) (layer "F.Cu") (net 11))
 (segment (start 145.6 107.25) (end 146.5625 107.25) (width 0.4) (locked yes) (layer "F.Cu") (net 11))
 (segment (start 148.575 107.25) (end 146.5625 107.25) (width 0.4) (locked yes) (layer "F.Cu") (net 11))
 (segment (start 131.2 97.2) (end 132.8 98.8) (width 0.4) (locked yes) (layer "F.Cu") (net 11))
 (segment (start 136 98.8) (end 136.125 98.675) (width 0.4) (locked yes) (layer "F.Cu") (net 11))
 (segment (start 126.55 97.2) (end 131.2 97.2) (width 0.4) (locked yes) (layer "F.Cu") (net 11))
 (segment (start 138.9125 98.3125) (end 139.55 98.95) (width 0.4) (locked yes) (layer "F.Cu") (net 11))
 (segment (start 148.8625 108.2) (end 148.8625 107.5375) (width 0.4) (locked yes) (layer "F.Cu") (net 11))
 (segment (start 137.2 98.3125) (end 138.9125 98.3125) (width 0.4) (locked yes) (layer "F.Cu") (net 11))
 (segment (start 139.55 105) (end 140.3 105.75) (width 0.4) (locked yes) (layer "F.Cu") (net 11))
 (segment (start 139.55 98.95) (end 139.55 105) (width 0.4) (locked yes) (layer "F.Cu") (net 11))
 (segment (start 132.8 98.8) (end 135.05 98.8) (width 0.4) (locked yes) (layer "F.Cu") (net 11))
 (segment (start 136.3 99.9) (end 137.0125 99.9) (width 0.2) (locked yes) (layer "F.Cu") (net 29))
 (segment (start 136 99.6) (end 136.125 99.725) (width 0.2) (locked yes) (layer "F.Cu") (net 29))
 (segment (start 137.0125 99.9) (end 137.2 100.0875) (width 0.2) (locked yes) (layer "F.Cu") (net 29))
 (segment (start 136.125 99.725) (end 136.3 99.9) (width 0.2) (locked yes) (layer "F.Cu") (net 29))
 (segment (start 135.05 99.6) (end 136 99.6) (width 0.2) (locked yes) (layer "F.Cu") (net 29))
 (segment (start 135.05 98) (end 133.2 98) (width 0.2) (locked yes) (layer "F.Cu") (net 30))
 (segment (start 133.2 98) (end 132.4 97.2) (width 0.2) (locked yes) (layer "F.Cu") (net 30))
 (via (at 132.4 97.2) (size 0.6) (drill 0.3) (layers "F.Cu" "B.Cu") (locked yes) (free yes) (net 30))
 (segment (start 133.6 97.2) (end 135.05 97.2) (width 0.2) (locked yes) (layer "F.Cu") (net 31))
 (via (at 133.6 97.2) (size 0.6) (drill 0.3) (layers "F.Cu" "B.Cu") (locked yes) (free yes) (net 31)))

